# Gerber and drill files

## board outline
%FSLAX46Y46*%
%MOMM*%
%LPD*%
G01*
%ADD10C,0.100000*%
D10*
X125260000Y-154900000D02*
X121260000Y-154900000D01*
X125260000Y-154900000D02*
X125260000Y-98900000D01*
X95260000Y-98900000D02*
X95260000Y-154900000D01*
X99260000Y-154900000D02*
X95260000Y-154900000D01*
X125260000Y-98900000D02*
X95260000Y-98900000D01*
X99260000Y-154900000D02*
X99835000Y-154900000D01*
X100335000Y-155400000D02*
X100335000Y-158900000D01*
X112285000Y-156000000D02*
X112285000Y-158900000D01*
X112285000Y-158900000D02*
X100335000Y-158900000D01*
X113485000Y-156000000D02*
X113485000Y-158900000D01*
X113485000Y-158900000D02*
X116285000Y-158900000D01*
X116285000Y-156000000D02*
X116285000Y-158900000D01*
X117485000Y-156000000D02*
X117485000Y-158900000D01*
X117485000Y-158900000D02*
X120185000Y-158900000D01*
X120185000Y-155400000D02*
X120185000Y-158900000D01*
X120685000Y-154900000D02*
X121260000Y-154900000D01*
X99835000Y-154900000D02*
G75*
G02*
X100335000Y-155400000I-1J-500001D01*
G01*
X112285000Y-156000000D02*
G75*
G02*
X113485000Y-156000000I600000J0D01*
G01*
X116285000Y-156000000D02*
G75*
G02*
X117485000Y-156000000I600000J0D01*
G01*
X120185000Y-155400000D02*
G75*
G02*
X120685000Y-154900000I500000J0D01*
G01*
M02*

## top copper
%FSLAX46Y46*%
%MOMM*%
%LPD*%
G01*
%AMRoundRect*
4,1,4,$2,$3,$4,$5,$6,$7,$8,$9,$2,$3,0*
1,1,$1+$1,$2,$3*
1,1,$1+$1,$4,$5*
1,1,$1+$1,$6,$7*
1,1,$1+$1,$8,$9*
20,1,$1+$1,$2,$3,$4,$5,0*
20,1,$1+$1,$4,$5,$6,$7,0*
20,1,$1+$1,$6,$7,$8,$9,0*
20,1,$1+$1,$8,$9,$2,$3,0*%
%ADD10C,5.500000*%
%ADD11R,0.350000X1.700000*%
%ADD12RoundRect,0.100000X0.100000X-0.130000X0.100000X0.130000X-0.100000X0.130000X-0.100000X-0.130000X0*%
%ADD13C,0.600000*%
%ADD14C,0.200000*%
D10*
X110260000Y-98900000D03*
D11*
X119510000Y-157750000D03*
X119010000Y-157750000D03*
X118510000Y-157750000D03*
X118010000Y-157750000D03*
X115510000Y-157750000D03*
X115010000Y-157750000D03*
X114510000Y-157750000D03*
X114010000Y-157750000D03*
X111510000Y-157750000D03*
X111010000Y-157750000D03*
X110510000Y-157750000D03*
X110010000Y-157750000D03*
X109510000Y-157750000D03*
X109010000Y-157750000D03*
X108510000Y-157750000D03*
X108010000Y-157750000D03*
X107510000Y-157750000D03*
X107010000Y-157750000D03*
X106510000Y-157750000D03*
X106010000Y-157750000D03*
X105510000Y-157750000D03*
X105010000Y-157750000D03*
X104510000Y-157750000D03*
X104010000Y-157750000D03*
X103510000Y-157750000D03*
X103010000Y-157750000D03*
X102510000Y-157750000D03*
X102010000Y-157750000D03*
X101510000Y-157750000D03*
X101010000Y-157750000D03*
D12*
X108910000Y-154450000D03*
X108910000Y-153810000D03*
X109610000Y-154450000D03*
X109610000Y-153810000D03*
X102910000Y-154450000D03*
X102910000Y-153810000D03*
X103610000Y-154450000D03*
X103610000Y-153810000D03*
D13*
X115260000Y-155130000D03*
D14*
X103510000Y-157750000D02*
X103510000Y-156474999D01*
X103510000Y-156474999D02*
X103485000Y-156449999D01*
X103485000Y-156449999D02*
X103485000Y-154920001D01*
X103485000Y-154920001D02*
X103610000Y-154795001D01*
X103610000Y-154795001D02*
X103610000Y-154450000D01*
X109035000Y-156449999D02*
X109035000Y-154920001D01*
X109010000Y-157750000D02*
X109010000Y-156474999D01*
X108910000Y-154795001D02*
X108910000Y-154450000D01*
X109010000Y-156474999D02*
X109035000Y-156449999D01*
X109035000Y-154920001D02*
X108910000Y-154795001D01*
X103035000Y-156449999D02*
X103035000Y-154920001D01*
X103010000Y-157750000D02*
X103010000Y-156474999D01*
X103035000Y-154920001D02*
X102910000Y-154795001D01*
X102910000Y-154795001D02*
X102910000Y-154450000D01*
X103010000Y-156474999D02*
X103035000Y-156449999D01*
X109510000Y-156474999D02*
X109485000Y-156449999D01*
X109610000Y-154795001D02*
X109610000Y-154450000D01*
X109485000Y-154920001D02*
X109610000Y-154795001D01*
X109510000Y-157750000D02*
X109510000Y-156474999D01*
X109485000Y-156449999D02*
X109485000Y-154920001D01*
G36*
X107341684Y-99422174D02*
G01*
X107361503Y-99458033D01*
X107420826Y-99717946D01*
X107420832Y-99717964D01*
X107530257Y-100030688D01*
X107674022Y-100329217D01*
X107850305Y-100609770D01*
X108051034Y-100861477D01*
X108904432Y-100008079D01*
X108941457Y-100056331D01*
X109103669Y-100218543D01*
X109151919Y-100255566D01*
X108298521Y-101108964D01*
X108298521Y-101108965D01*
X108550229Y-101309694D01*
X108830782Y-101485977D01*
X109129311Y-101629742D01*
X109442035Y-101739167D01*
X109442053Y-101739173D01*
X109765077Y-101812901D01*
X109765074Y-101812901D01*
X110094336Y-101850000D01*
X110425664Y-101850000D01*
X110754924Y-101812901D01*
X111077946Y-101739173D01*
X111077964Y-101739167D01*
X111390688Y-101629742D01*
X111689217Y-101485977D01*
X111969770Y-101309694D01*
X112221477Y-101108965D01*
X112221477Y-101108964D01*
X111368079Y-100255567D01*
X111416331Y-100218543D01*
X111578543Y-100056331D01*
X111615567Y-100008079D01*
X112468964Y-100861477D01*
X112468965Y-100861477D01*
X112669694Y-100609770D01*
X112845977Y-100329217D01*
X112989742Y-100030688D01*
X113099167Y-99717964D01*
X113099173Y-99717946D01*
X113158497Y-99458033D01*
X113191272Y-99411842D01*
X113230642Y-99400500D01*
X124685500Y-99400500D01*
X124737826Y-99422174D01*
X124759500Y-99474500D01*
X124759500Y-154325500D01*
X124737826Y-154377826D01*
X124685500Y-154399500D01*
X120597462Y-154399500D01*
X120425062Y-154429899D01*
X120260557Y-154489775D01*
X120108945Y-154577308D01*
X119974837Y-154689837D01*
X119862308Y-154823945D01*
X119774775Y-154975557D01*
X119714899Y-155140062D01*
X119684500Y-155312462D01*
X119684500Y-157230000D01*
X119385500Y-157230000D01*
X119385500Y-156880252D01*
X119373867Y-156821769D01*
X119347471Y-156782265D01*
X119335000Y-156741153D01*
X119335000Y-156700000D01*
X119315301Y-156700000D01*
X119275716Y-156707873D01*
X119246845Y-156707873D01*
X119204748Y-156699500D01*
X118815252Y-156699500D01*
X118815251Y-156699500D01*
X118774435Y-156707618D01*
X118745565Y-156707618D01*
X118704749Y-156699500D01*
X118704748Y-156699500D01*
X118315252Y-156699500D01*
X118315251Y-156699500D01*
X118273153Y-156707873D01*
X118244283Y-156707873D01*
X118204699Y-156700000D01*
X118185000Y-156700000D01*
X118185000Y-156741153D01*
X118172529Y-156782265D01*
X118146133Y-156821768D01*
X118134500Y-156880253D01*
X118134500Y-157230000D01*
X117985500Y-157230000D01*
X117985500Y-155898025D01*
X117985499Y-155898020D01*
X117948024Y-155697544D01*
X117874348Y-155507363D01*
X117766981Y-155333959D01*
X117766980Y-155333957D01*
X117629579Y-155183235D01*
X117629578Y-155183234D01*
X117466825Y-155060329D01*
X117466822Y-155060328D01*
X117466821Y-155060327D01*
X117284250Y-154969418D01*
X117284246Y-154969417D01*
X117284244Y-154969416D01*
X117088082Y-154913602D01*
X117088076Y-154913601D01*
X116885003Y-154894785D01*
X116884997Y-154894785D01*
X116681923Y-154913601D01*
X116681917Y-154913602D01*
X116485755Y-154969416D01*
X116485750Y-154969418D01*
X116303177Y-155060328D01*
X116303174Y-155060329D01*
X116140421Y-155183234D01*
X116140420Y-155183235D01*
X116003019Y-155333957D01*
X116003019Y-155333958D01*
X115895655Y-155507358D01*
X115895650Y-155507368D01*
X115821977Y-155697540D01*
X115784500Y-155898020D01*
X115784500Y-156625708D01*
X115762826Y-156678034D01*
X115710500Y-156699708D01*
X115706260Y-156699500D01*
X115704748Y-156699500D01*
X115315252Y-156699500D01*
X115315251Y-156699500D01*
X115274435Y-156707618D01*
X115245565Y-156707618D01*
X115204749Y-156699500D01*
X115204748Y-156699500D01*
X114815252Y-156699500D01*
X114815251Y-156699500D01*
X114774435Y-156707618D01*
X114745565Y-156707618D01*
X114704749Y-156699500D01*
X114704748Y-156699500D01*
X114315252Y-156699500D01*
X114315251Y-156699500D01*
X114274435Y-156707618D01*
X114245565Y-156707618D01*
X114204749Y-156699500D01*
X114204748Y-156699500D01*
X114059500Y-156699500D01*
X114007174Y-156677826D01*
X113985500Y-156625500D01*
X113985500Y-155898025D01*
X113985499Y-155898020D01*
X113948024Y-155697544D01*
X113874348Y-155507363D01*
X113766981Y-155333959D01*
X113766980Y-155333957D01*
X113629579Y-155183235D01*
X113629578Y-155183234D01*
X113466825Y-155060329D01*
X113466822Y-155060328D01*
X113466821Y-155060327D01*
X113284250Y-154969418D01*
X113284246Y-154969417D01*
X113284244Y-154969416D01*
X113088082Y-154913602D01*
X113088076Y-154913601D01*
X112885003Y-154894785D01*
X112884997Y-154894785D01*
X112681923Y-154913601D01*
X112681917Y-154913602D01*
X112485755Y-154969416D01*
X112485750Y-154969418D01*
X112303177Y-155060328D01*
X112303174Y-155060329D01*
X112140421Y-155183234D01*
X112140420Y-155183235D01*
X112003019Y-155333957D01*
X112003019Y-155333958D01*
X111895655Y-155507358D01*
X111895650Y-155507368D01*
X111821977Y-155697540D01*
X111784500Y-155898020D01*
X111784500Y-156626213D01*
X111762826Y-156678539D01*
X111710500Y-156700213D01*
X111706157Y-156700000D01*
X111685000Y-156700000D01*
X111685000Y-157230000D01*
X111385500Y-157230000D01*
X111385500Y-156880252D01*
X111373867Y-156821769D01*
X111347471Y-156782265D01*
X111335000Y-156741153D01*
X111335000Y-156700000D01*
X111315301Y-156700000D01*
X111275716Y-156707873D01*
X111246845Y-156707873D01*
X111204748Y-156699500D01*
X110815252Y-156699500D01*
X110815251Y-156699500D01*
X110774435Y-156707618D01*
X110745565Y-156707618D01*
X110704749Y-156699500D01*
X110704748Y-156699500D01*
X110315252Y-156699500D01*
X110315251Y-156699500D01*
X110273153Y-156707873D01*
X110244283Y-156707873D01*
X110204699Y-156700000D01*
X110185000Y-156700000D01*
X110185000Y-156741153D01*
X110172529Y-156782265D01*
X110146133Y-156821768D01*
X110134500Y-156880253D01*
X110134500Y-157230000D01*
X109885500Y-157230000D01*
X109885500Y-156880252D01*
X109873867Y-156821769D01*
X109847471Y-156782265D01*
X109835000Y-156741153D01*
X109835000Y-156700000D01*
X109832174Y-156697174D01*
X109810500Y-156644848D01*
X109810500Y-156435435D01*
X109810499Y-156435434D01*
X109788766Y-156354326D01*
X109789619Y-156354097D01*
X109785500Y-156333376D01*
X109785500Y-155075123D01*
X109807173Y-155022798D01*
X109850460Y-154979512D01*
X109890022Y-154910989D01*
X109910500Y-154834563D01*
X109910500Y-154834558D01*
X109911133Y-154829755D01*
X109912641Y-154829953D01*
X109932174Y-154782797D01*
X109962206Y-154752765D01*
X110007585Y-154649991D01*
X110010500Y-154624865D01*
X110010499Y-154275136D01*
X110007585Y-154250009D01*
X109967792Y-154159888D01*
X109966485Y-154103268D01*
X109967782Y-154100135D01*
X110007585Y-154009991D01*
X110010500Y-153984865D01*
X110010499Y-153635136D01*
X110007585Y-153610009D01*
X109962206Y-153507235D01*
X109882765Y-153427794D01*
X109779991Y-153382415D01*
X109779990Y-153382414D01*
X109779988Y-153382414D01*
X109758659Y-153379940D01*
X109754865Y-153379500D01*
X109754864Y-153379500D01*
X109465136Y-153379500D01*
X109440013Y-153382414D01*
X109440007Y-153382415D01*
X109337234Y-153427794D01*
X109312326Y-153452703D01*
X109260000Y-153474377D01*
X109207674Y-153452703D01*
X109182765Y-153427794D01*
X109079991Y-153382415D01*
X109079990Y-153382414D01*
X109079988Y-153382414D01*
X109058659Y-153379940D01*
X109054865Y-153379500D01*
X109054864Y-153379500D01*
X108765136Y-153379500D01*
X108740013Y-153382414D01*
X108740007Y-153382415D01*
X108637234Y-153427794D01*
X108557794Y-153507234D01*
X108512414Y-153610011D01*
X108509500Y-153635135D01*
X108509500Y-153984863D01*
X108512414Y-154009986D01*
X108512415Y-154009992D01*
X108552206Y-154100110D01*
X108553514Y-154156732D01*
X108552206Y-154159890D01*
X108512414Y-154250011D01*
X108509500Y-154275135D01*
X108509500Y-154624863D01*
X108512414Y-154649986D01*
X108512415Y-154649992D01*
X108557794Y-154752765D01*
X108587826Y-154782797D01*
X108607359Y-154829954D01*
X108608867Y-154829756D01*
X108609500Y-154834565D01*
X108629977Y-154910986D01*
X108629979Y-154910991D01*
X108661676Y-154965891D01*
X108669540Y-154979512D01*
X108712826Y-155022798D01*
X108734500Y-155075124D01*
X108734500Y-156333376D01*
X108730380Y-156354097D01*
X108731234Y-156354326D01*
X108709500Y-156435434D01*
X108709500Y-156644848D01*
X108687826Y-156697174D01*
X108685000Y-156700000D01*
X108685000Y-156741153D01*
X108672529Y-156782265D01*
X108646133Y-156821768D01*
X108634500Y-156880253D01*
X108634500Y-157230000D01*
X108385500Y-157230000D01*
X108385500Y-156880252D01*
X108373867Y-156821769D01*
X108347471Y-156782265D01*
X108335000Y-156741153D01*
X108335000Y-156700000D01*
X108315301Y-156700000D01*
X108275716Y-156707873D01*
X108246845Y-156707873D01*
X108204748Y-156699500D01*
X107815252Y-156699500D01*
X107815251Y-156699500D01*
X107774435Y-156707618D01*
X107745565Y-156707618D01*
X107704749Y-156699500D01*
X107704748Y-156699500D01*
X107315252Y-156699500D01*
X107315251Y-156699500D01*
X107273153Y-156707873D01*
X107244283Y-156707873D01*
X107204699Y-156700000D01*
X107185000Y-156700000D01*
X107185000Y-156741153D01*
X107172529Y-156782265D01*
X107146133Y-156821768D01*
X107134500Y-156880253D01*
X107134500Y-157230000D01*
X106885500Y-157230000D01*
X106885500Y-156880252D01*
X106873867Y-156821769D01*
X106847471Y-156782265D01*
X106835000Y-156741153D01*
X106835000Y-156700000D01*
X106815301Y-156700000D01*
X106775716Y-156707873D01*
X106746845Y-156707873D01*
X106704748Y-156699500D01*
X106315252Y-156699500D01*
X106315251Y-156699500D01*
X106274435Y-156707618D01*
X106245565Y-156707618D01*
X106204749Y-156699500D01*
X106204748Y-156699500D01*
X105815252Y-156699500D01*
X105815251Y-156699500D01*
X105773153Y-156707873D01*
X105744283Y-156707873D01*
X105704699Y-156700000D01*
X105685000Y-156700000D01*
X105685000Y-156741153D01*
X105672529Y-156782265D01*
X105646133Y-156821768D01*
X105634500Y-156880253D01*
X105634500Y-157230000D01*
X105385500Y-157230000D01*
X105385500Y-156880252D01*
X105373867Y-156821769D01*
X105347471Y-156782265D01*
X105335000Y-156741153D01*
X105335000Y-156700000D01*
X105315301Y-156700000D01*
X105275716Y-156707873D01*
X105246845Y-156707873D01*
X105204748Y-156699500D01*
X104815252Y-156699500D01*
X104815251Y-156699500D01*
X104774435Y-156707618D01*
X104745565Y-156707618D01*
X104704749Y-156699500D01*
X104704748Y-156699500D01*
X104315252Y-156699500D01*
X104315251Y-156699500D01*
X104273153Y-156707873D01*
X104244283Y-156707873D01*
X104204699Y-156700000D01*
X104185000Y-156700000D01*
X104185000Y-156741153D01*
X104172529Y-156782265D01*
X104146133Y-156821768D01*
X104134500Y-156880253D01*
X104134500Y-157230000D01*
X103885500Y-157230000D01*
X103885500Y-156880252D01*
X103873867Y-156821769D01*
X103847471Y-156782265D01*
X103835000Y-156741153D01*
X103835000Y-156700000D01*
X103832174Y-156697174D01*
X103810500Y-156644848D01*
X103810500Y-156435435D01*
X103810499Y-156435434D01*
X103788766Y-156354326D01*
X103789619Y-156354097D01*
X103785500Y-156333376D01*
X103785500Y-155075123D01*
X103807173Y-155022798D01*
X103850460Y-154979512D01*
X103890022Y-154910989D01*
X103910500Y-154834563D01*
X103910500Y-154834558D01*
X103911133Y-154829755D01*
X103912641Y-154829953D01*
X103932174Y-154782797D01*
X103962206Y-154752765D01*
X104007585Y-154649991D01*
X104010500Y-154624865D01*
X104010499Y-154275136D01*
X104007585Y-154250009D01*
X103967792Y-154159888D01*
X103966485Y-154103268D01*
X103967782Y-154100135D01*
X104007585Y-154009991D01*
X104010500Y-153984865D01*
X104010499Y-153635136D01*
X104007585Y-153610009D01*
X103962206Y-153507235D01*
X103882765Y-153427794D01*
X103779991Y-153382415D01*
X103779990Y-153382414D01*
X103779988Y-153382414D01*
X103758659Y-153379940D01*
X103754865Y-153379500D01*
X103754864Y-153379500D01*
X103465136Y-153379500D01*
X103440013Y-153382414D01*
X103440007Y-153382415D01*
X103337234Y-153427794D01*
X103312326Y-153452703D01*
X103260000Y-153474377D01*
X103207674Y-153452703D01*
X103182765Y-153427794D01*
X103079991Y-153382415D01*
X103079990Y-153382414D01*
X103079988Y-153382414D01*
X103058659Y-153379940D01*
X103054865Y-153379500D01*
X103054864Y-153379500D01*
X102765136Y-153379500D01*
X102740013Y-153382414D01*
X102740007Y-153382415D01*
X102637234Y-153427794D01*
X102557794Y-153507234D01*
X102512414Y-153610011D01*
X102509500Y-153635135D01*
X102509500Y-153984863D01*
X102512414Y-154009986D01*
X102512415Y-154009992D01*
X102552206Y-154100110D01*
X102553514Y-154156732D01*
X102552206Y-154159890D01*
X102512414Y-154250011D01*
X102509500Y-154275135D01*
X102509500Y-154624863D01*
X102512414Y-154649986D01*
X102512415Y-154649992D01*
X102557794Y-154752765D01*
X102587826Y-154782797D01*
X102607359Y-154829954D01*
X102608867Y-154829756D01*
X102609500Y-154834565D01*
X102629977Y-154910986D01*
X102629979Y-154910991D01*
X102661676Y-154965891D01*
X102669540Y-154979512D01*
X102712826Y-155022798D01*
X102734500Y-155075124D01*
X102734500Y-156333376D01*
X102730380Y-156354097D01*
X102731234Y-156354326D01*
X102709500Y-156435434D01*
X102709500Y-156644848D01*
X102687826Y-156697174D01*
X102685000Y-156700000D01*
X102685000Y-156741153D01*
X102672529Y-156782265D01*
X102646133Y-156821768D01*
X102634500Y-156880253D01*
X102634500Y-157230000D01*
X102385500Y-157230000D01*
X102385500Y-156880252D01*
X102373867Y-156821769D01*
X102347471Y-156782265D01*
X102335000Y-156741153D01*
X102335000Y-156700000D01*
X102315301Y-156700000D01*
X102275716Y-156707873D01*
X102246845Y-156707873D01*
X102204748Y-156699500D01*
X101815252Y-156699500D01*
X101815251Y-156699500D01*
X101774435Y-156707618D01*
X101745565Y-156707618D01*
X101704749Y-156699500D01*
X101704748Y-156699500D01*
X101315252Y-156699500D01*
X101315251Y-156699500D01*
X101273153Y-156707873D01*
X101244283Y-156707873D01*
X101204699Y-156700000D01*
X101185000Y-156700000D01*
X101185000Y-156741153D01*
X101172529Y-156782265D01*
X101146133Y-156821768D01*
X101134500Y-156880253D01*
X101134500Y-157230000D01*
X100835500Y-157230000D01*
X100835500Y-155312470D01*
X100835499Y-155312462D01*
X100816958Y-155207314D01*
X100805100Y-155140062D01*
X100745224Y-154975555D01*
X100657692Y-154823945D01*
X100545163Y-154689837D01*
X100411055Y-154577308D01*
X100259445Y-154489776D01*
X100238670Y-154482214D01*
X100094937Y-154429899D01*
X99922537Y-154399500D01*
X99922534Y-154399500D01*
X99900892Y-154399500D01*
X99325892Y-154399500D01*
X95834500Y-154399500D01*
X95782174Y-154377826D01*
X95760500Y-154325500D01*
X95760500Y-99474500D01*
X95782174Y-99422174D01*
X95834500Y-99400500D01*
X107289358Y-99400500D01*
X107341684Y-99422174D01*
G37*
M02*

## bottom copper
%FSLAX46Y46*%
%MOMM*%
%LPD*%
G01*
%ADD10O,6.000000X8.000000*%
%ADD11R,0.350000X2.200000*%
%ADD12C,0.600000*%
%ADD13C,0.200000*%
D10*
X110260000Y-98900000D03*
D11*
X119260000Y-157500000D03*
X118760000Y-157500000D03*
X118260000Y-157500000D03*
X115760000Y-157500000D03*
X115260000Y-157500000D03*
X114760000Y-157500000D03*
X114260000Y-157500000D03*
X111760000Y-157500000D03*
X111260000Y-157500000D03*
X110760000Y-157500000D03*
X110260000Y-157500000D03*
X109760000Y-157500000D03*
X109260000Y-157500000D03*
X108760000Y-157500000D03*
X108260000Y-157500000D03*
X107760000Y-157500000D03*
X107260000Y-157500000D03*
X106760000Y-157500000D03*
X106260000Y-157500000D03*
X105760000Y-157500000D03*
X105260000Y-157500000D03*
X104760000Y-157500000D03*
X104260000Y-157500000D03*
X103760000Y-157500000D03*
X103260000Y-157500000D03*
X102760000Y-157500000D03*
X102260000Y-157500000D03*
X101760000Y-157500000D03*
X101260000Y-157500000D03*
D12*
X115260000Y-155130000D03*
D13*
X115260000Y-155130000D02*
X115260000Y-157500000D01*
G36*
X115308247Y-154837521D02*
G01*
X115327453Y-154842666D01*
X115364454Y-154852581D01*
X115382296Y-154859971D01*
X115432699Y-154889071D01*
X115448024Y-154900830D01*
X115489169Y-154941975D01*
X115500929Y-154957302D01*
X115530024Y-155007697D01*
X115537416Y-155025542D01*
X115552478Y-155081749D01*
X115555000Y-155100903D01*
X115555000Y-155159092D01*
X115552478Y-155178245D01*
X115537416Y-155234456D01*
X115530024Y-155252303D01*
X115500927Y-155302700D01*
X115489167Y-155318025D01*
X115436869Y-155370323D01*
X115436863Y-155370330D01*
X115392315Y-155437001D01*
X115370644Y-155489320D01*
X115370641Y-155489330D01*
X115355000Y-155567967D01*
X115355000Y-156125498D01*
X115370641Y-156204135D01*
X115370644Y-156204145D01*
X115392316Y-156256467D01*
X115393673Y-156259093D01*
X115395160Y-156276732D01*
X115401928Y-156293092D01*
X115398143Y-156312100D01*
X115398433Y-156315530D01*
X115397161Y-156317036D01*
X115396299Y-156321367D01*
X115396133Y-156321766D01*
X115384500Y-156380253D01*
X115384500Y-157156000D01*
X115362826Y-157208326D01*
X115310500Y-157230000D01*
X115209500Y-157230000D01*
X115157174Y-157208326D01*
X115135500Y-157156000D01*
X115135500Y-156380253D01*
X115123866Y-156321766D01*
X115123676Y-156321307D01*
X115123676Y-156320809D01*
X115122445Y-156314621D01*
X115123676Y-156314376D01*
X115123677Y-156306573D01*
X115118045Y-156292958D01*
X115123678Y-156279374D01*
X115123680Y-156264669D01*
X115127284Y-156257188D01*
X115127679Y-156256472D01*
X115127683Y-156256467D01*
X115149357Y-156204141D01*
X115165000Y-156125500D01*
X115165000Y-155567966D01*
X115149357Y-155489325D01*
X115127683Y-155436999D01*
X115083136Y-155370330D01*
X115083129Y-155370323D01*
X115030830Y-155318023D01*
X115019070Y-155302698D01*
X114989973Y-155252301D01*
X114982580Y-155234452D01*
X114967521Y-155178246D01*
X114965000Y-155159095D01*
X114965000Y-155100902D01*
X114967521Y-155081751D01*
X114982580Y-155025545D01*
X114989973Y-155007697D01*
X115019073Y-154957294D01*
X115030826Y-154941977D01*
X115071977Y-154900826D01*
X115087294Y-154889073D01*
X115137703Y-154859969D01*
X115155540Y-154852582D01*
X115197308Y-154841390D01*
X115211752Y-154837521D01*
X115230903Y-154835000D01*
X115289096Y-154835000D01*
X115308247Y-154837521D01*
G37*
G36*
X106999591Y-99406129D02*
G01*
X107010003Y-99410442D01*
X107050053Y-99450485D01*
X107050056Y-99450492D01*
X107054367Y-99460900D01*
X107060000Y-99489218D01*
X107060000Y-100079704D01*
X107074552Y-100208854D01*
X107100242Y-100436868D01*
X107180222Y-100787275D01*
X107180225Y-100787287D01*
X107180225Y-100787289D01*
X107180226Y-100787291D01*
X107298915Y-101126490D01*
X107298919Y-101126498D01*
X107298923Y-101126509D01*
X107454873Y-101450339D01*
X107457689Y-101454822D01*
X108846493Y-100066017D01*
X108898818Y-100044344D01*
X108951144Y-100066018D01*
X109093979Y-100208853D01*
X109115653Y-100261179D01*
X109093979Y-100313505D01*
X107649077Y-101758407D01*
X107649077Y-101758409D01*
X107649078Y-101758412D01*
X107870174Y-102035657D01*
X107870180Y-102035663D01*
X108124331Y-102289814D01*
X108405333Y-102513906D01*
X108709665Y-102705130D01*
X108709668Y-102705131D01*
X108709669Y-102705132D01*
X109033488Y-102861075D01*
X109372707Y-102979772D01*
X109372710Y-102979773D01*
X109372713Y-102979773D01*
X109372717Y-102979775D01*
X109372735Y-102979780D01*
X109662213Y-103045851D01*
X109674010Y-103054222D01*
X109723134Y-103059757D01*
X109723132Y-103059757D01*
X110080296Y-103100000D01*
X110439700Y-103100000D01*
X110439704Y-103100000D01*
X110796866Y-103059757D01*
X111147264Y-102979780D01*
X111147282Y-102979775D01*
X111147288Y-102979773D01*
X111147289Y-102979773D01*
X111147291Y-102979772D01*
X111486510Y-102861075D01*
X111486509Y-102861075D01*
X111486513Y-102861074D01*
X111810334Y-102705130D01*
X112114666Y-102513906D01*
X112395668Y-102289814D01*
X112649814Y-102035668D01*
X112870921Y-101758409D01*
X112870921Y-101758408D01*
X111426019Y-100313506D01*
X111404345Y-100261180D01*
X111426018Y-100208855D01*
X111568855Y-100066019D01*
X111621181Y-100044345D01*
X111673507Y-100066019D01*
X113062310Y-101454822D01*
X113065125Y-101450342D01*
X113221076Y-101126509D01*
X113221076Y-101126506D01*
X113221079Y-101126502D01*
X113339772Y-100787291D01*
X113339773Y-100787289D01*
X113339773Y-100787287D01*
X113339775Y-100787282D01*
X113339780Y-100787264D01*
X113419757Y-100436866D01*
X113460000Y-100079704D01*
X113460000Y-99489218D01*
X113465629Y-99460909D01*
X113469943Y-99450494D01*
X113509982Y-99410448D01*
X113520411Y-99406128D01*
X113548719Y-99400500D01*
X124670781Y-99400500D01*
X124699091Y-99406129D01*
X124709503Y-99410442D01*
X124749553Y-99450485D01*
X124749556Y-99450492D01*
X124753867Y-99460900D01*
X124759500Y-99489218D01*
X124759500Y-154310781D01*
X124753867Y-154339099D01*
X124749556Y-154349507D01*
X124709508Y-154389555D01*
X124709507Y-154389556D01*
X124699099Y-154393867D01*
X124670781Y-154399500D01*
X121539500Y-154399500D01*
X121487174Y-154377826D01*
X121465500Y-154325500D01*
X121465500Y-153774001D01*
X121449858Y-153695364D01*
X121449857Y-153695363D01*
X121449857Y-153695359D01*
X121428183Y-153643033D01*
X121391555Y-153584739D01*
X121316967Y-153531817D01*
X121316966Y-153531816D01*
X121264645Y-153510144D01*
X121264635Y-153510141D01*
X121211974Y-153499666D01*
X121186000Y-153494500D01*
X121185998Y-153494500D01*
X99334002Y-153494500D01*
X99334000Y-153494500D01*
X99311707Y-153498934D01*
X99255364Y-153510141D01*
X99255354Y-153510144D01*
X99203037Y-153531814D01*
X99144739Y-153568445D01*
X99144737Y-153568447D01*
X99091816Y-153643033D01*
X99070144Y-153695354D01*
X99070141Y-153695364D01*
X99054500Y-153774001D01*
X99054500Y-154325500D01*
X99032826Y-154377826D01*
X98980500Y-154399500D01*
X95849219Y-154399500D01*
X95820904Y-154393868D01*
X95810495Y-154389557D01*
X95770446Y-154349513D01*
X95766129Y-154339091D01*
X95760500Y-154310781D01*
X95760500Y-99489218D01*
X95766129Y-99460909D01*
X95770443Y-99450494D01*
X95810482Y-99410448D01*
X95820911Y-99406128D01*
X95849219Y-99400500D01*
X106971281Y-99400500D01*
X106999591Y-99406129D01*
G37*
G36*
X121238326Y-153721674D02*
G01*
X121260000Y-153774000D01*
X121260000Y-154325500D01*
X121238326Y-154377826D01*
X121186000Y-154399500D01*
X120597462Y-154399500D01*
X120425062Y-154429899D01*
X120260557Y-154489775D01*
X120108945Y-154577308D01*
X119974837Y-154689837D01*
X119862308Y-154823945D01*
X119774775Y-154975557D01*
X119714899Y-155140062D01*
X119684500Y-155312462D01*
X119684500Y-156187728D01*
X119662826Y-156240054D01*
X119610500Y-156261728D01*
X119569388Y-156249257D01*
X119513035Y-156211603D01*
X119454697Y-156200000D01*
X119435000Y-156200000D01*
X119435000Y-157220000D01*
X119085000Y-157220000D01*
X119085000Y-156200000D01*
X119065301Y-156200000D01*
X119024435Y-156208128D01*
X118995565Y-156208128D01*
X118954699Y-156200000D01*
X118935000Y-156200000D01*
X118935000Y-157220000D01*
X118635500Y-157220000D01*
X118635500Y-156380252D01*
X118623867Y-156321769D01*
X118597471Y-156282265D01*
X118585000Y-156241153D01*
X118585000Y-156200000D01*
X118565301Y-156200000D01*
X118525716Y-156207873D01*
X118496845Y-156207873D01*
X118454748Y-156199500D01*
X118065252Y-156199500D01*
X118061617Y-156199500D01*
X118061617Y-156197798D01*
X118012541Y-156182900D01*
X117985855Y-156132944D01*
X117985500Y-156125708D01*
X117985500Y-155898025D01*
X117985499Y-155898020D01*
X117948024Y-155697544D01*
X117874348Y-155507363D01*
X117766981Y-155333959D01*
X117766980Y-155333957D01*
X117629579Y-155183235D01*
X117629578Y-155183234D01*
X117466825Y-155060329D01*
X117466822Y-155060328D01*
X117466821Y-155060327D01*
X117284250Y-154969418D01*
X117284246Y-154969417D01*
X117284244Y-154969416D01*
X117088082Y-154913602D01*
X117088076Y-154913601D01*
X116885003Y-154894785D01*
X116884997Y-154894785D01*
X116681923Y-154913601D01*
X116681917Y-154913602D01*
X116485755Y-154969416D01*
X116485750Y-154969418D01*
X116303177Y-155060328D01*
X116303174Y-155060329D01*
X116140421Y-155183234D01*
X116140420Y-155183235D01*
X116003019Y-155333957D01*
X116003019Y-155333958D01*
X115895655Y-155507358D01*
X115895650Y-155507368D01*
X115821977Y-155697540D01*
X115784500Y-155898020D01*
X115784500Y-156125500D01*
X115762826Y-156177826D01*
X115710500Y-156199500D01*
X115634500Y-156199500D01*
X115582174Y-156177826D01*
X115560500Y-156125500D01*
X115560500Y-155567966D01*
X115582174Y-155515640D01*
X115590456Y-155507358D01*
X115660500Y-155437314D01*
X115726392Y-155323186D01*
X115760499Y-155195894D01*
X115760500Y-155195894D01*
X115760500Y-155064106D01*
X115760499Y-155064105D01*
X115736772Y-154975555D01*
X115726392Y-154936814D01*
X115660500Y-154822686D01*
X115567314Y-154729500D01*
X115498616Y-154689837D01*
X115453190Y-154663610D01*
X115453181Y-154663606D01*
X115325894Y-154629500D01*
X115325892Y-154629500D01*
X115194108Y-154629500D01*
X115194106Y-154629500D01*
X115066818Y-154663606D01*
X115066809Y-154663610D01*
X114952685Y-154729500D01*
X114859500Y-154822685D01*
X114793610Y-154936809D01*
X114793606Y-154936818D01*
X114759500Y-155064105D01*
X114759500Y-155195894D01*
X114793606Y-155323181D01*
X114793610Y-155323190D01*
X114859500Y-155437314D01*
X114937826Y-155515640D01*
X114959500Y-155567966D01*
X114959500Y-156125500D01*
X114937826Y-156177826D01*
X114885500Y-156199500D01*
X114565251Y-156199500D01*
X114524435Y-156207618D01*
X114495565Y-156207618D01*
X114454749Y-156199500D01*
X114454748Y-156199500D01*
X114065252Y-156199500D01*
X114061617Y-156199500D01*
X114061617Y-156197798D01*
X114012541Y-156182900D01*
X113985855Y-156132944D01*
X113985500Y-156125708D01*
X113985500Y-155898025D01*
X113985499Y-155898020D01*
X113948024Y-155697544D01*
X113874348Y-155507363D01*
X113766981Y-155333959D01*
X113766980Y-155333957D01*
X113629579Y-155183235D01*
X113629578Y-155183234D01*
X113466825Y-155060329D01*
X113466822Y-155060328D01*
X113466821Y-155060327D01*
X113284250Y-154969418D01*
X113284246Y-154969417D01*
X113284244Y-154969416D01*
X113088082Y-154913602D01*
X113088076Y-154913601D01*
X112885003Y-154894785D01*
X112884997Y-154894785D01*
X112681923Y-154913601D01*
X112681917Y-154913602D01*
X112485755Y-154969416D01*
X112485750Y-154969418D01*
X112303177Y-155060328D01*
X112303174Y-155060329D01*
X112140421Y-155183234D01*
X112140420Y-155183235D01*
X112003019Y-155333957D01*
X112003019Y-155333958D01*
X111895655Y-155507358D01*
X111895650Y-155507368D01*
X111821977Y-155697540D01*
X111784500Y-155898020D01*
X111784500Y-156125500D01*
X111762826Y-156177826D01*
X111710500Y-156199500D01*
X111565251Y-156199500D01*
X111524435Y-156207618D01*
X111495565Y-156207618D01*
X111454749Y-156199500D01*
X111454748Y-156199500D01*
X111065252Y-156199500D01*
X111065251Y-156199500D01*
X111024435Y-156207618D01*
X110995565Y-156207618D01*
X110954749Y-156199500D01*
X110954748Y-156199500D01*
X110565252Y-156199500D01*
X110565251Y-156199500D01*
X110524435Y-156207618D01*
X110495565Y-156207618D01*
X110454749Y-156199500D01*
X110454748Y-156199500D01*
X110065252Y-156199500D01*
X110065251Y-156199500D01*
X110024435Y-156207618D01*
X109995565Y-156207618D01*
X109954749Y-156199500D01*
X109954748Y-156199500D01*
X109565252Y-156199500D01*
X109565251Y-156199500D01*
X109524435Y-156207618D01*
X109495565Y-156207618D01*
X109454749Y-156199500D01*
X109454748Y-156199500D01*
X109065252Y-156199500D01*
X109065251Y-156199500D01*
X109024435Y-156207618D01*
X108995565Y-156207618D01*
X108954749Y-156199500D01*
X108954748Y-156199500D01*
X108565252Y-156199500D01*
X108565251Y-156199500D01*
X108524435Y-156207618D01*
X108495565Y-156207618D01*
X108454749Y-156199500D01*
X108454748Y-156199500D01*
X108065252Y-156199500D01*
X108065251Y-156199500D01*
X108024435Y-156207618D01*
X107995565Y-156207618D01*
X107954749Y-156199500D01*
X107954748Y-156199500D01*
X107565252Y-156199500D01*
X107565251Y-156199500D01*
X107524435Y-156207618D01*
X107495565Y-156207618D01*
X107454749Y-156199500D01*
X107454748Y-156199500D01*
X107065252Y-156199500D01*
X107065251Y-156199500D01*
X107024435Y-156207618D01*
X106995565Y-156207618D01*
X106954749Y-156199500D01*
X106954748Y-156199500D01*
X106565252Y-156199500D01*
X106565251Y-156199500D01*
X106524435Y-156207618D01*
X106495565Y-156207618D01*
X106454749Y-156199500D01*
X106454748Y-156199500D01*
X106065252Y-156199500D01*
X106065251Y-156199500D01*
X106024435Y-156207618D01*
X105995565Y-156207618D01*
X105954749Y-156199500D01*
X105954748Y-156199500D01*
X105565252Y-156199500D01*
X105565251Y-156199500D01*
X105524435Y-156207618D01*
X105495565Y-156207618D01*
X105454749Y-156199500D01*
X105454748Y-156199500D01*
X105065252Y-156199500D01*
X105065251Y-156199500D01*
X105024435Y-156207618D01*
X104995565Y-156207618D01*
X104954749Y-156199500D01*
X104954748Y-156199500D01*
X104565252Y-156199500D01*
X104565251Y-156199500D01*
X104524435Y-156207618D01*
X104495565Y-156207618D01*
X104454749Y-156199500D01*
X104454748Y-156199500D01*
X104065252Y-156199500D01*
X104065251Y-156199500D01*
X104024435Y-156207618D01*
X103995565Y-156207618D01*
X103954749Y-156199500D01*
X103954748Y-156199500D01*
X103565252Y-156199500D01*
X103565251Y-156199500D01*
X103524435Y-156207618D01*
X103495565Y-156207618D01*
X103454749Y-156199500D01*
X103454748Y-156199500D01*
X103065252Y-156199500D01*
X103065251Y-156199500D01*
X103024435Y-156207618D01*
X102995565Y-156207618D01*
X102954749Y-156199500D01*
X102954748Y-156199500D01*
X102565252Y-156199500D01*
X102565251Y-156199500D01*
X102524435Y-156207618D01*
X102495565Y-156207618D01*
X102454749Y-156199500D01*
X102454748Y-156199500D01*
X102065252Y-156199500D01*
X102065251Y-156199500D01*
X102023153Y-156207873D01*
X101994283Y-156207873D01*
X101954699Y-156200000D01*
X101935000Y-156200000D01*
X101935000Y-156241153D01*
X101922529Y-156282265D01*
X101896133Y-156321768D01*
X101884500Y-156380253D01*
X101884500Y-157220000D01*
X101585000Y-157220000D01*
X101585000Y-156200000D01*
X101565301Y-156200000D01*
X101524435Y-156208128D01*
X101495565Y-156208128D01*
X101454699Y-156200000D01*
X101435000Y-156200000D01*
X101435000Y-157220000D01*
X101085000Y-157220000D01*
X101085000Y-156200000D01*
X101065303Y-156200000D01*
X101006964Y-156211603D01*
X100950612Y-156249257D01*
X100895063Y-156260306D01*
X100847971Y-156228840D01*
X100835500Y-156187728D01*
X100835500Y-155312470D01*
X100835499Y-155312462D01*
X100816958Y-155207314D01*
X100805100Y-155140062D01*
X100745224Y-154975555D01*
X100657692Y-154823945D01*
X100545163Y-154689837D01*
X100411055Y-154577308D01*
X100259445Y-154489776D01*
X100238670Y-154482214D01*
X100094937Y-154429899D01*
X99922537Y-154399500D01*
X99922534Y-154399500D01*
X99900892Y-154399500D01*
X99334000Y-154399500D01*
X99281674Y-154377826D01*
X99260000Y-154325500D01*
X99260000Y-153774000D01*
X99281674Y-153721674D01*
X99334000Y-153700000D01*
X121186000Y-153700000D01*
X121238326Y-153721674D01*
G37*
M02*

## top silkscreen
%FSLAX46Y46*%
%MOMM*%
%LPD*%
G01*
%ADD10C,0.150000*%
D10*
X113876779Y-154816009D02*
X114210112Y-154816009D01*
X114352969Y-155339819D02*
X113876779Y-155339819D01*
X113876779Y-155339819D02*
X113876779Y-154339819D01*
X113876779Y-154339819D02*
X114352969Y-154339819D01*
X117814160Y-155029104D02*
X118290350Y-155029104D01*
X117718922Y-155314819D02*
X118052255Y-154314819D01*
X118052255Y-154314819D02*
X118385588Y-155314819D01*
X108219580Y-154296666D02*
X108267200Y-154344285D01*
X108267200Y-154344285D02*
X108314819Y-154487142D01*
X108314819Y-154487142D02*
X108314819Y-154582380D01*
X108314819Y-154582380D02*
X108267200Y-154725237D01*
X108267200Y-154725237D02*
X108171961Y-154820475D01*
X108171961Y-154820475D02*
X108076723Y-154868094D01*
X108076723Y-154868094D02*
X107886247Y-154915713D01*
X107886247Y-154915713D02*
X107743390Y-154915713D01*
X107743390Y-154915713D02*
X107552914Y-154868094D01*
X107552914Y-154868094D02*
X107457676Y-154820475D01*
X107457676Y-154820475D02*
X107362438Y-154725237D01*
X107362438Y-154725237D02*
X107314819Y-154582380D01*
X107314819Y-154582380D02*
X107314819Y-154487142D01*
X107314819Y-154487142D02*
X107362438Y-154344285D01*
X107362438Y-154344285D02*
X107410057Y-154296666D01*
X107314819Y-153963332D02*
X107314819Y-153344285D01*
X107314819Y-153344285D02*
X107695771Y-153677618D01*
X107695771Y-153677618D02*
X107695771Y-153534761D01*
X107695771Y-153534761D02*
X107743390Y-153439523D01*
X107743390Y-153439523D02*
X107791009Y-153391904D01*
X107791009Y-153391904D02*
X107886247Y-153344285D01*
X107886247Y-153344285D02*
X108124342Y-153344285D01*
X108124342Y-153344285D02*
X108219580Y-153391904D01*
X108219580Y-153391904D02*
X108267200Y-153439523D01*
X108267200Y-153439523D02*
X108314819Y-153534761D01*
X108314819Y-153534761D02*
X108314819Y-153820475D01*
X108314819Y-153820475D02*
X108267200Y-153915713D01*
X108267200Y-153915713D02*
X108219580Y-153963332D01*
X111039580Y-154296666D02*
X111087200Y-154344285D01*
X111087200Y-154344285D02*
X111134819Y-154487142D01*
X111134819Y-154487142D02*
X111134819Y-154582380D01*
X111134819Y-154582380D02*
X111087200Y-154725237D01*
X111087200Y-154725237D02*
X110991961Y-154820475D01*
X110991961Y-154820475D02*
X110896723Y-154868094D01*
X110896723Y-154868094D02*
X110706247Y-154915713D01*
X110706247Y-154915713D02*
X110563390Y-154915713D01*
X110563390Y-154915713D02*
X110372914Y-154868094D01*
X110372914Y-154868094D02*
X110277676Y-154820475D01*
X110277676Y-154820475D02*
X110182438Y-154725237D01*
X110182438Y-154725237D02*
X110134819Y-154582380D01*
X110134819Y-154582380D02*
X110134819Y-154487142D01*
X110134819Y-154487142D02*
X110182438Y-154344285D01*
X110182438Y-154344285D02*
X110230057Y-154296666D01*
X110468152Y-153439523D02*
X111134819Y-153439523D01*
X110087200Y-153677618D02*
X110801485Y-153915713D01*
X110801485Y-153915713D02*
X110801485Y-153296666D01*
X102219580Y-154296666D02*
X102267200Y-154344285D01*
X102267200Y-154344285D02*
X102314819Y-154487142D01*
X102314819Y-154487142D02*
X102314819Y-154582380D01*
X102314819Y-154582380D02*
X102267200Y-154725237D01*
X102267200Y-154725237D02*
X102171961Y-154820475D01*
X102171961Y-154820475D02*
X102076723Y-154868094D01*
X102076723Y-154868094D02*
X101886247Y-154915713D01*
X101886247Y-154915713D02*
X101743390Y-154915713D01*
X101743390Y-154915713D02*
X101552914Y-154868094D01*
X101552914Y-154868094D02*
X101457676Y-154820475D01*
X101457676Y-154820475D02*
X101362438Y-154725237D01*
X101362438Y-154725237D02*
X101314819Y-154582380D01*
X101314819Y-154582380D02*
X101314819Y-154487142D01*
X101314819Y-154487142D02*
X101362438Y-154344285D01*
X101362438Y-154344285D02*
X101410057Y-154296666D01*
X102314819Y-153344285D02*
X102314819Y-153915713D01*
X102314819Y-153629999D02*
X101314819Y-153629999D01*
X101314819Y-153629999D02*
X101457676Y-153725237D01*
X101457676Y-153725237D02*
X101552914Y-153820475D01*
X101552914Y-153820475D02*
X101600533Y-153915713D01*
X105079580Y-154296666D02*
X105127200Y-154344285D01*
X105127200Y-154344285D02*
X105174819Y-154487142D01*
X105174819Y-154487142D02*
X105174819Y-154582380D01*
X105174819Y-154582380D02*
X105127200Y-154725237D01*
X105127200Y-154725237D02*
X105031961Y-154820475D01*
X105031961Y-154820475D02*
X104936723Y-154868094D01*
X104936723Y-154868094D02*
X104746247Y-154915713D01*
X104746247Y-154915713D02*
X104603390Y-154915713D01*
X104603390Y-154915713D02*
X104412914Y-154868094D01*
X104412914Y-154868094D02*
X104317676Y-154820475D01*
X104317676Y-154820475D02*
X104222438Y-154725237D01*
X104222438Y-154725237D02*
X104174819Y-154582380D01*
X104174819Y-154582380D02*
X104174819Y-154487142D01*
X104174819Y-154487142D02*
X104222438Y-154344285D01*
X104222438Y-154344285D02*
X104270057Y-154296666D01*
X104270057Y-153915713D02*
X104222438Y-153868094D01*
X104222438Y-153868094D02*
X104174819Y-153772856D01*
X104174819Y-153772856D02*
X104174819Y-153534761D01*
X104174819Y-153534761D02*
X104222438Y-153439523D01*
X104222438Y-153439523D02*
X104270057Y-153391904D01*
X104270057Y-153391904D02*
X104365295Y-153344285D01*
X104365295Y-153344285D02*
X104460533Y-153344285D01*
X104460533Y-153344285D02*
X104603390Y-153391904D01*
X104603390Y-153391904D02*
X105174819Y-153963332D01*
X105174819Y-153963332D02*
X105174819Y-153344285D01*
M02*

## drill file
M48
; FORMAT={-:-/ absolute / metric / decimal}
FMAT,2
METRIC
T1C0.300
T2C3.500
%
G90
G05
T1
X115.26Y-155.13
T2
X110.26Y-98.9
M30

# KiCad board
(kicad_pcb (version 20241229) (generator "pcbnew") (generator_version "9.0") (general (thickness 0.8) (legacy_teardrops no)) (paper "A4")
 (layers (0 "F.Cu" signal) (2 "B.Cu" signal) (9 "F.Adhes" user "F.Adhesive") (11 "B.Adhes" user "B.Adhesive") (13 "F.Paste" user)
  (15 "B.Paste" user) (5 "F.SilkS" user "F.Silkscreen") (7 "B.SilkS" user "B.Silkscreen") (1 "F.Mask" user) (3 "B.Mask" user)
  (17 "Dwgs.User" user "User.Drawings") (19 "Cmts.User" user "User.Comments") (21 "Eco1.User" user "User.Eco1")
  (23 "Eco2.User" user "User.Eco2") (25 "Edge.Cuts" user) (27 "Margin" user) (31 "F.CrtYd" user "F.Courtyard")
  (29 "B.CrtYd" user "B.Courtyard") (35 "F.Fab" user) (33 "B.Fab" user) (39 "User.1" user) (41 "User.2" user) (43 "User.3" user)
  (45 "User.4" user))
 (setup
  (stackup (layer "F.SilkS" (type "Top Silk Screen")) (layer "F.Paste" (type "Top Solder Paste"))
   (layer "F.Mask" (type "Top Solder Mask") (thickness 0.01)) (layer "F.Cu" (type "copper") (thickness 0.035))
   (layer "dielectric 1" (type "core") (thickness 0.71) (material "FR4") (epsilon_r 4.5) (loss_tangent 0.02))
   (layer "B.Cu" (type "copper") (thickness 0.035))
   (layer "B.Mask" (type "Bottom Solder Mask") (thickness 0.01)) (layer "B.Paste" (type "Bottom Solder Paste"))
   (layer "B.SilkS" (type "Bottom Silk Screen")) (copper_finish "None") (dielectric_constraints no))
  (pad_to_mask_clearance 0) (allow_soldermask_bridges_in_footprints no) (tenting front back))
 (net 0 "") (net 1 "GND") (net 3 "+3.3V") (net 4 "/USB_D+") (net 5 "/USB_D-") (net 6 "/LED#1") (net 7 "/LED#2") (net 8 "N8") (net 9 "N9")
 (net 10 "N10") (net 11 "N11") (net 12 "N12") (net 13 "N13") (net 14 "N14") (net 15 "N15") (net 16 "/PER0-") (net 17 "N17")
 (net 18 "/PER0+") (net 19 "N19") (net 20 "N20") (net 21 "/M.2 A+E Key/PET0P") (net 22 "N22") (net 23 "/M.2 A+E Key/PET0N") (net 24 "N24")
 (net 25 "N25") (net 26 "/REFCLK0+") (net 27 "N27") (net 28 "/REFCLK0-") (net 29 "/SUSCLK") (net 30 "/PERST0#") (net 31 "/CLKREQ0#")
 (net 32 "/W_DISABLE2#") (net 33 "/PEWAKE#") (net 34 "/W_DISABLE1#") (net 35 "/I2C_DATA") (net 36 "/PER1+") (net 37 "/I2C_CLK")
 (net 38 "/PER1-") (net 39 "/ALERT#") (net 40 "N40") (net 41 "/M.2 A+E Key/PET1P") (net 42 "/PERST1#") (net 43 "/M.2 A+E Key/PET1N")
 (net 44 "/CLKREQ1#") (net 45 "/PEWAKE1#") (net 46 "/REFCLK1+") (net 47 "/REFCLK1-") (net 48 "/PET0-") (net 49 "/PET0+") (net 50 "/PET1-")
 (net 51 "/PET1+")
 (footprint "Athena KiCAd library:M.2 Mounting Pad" (layer "F.Cu") (at 110.26 98.9)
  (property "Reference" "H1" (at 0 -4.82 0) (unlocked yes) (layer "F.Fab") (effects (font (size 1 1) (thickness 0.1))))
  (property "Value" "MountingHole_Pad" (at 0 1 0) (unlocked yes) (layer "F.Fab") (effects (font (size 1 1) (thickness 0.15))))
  (pad "1" thru_hole circle (at 0 0) (size 5.5 5.5) (drill 3.5) (layers "*.Cu" "*.Mask") (remove_unused_layers no) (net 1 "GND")
   (padstack (mode front_inner_back)
    (layer "Inner" (shape circle) (size 5.5 5.5) (zone_connect -1))
    (layer "B.Cu" (shape oval) (size 6 8) (thermal_bridge_angle 45) (zone_connect -1)))))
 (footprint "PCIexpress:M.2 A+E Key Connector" (layer "F.Cu") (at 110.26 157.79)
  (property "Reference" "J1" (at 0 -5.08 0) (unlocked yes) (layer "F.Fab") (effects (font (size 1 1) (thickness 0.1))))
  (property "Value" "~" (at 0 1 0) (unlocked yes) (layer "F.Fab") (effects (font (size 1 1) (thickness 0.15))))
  (fp_line (start -11 -2.89) (end -10.425 -2.89) (stroke (width 0.1) (type default)) (layer "Edge.Cuts") (net 2))
  (fp_line (start -9.925 -2.39) (end -9.925 1.11) (stroke (width 0.1) (type default)) (layer "Edge.Cuts") (net 2))
  (fp_line (start 2.025 -1.79) (end 2.025 1.11) (stroke (width 0.1) (type default)) (layer "Edge.Cuts") (net 2))
  (fp_line (start 2.025 1.11) (end -9.925 1.11) (stroke (width 0.1) (type default)) (layer "Edge.Cuts") (net 2))
  (fp_line (start 3.225 -1.79) (end 3.225 1.11) (stroke (width 0.1) (type default)) (layer "Edge.Cuts") (net 2))
  (fp_line (start 3.225 1.11) (end 6.025 1.11) (stroke (width 0.1) (type default)) (layer "Edge.Cuts") (net 2))
  (fp_line (start 6.025 -1.79) (end 6.025 1.11) (stroke (width 0.1) (type default)) (layer "Edge.Cuts") (net 2))
  (fp_line (start 7.225 -1.79) (end 7.225 1.11) (stroke (width 0.1) (type default)) (layer "Edge.Cuts") (net 2))
  (fp_line (start 7.225 1.11) (end 9.925 1.11) (stroke (width 0.1) (type default)) (layer "Edge.Cuts") (net 2))
  (fp_line (start 9.925 -2.39) (end 9.925 1.11) (stroke (width 0.1) (type default)) (layer "Edge.Cuts") (net 2))
  (fp_line (start 10.425 -2.89) (end 11 -2.89) (stroke (width 0.1) (type default)) (layer "Edge.Cuts") (net 2))
  (fp_arc (start -10.425 -2.89) (mid -10.071447 -2.743553) (end -9.925 -2.39) (stroke (width 0.1) (type default)) (layer "Edge.Cuts")
   (net 2))
  (fp_arc (start 2.025 -1.79) (mid 2.625 -2.39) (end 3.225 -1.79) (stroke (width 0.1) (type default)) (layer "Edge.Cuts") (net 2))
  (fp_arc (start 6.025 -1.79) (mid 6.625 -2.39) (end 7.225 -1.79) (stroke (width 0.1) (type default)) (layer "Edge.Cuts") (net 2))
  (fp_arc (start 9.925 -2.39) (mid 10.071447 -2.743553) (end 10.425 -2.89) (stroke (width 0.1) (type default)) (layer "Edge.Cuts") (net 2))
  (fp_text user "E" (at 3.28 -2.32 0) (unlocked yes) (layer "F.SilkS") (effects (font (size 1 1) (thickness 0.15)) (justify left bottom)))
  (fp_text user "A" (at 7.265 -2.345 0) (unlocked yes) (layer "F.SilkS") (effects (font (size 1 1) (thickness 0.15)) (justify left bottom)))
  (pad "1" smd rect (at 9.25 -0.04 180) (size 0.35 1.7) (layers "F.Cu") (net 1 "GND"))
  (pad "2" smd rect (at 9 -0.29 180) (size 0.35 2.2) (layers "B.Cu") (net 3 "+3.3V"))
  (pad "3" smd rect (at 8.75 -0.04 180) (size 0.35 1.7) (layers "F.Cu") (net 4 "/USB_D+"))
  (pad "4" smd rect (at 8.5 -0.29 180) (size 0.35 2.2) (layers "B.Cu") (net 3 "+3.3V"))
  (pad "5" smd rect (at 8.25 -0.04 180) (size 0.35 1.7) (layers "F.Cu") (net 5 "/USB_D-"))
  (pad "6" smd rect (at 8 -0.29 180) (size 0.35 2.2) (layers "B.Cu") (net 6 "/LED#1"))
  (pad "7" smd rect (at 7.75 -0.04 180) (size 0.35 1.7) (layers "F.Cu") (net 1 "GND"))
  (pad "16" smd rect (at 5.5 -0.29 180) (size 0.35 2.2) (layers "B.Cu") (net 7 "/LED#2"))
  (pad "17" smd rect (at 5.25 -0.04 180) (size 0.35 1.7) (layers "F.Cu") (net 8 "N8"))
  (pad "18" smd rect (at 5 -0.29 180) (size 0.35 2.2) (layers "B.Cu") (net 1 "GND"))
  (pad "19" smd rect (at 4.75 -0.04 180) (size 0.35 1.7) (layers "F.Cu") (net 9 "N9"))
  (pad "20" smd rect (at 4.5 -0.29 180) (size 0.35 2.2) (layers "B.Cu") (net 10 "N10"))
  (pad "21" smd rect (at 4.25 -0.04 180) (size 0.35 1.7) (layers "F.Cu") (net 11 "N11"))
  (pad "22" smd rect (at 4 -0.29 180) (size 0.35 2.2) (layers "B.Cu") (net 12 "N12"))
  (pad "23" smd rect (at 3.75 -0.04 180) (size 0.35 1.7) (layers "F.Cu") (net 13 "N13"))
  (pad "32" smd rect (at 1.5 -0.29 180) (size 0.35 2.2) (layers "B.Cu") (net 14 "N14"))
  (pad "33" smd rect (at 1.25 -0.04 180) (size 0.35 1.7) (layers "F.Cu") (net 1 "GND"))
  (pad "34" smd rect (at 1 -0.29 180) (size 0.35 2.2) (layers "B.Cu") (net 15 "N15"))
  (pad "35" smd rect (at 0.75 -0.04 180) (size 0.35 1.7) (layers "F.Cu") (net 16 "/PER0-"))
  (pad "36" smd rect (at 0.5 -0.29 180) (size 0.35 2.2) (layers "B.Cu") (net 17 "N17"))
  (pad "37" smd rect (at 0.25 -0.04 180) (size 0.35 1.7) (layers "F.Cu") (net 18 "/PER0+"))
  (pad "38" smd rect (at 0 -0.29 180) (size 0.35 2.2) (layers "B.Cu") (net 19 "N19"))
  (pad "39" smd rect (at -0.25 -0.04 180) (size 0.35 1.7) (layers "F.Cu") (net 1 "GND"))
  (pad "40" smd rect (at -0.5 -0.29 180) (size 0.35 2.2) (layers "B.Cu") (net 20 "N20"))
  (pad "41" smd rect (at -0.75 -0.04 180) (size 0.35 1.7) (layers "F.Cu") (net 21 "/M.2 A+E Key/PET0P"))
  (pad "42" smd rect (at -1 -0.29 180) (size 0.35 2.2) (layers "B.Cu") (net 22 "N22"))
  (pad "43" smd rect (at -1.25 -0.04 180) (size 0.35 1.7) (layers "F.Cu") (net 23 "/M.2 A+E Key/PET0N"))
  (pad "44" smd rect (at -1.5 -0.29 180) (size 0.35 2.2) (layers "B.Cu") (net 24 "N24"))
  (pad "45" smd rect (at -1.75 -0.04 180) (size 0.35 1.7) (layers "F.Cu") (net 1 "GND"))
  (pad "46" smd rect (at -2 -0.29 180) (size 0.35 2.2) (layers "B.Cu") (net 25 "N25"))
  (pad "47" smd rect (at -2.25 -0.04 180) (size 0.35 1.7) (layers "F.Cu") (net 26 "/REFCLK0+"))
  (pad "48" smd rect (at -2.5 -0.29 180) (size 0.35 2.2) (layers "B.Cu") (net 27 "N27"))
  (pad "49" smd rect (at -2.75 -0.04 180) (size 0.35 1.7) (layers "F.Cu") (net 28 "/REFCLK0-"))
  (pad "50" smd rect (at -3 -0.29 180) (size 0.35 2.2) (layers "B.Cu") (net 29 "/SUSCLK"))
  (pad "51" smd rect (at -3.25 -0.04 180) (size 0.35 1.7) (layers "F.Cu") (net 1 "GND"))
  (pad "52" smd rect (at -3.5 -0.29 180) (size 0.35 2.2) (layers "B.Cu") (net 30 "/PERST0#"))
  (pad "53" smd rect (at -3.75 -0.04 180) (size 0.35 1.7) (layers "F.Cu") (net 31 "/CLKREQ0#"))
  (pad "54" smd rect (at -4 -0.29 180) (size 0.35 2.2) (layers "B.Cu") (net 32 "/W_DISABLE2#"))
  (pad "55" smd rect (at -4.25 -0.04 180) (size 0.35 1.7) (layers "F.Cu") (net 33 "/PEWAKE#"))
  (pad "56" smd rect (at -4.5 -0.29 180) (size 0.35 2.2) (layers "B.Cu") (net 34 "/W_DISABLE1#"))
  (pad "57" smd rect (at -4.75 -0.04 180) (size 0.35 1.7) (layers "F.Cu") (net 1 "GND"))
  (pad "58" smd rect (at -5 -0.29 180) (size 0.35 2.2) (layers "B.Cu") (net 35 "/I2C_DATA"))
  (pad "59" smd rect (at -5.25 -0.04 180) (size 0.35 1.7) (layers "F.Cu") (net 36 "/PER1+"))
  (pad "60" smd rect (at -5.5 -0.29 180) (size 0.35 2.2) (layers "B.Cu") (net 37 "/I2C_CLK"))
  (pad "61" smd rect (at -5.75 -0.04 180) (size 0.35 1.7) (layers "F.Cu") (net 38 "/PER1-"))
  (pad "62" smd rect (at -6 -0.29 180) (size 0.35 2.2) (layers "B.Cu") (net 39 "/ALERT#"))
  (pad "63" smd rect (at -6.25 -0.04 180) (size 0.35 1.7) (layers "F.Cu") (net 1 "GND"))
  (pad "64" smd rect (at -6.5 -0.29 180) (size 0.35 2.2) (layers "B.Cu") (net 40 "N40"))
  (pad "65" smd rect (at -6.75 -0.04 180) (size 0.35 1.7) (layers "F.Cu") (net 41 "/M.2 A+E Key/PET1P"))
  (pad "66" smd rect (at -7 -0.29 180) (size 0.35 2.2) (layers "B.Cu") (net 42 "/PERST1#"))
  (pad "67" smd rect (at -7.25 -0.04 180) (size 0.35 1.7) (layers "F.Cu") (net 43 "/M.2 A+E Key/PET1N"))
  (pad "68" smd rect (at -7.5 -0.29 180) (size 0.35 2.2) (layers "B.Cu") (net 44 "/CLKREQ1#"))
  (pad "69" smd rect (at -7.75 -0.04 180) (size 0.35 1.7) (layers "F.Cu") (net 1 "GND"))
  (pad "70" smd rect (at -8 -0.29 180) (size 0.35 2.2) (layers "B.Cu") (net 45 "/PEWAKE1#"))
  (pad "71" smd rect (at -8.25 -0.04 180) (size 0.35 1.7) (layers "F.Cu") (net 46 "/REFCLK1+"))
  (pad "72" smd rect (at -8.5 -0.29 180) (size 0.35 2.2) (layers "B.Cu") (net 3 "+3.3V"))
  (pad "73" smd rect (at -8.75 -0.04 180) (size 0.35 1.7) (layers "F.Cu") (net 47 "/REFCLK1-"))
  (pad "74" smd rect (at -9 -0.29 180) (size 0.35 2.2) (layers "B.Cu") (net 3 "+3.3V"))
  (pad "75" smd rect (at -9.25 -0.04 180) (size 0.35 1.7) (layers "F.Cu") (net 1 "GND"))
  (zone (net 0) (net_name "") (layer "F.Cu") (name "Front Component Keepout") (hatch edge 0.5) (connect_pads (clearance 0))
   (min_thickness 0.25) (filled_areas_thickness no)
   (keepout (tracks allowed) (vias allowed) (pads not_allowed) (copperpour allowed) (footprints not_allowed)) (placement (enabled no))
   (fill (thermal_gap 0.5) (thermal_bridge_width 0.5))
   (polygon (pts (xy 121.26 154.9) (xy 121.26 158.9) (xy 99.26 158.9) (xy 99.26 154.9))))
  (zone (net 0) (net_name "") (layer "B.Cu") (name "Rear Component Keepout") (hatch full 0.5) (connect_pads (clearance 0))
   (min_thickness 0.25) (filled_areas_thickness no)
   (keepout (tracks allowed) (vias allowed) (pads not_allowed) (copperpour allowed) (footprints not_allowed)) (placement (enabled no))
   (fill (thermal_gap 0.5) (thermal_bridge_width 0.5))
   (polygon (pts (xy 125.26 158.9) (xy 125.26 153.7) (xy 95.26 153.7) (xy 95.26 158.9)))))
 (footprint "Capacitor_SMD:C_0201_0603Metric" (layer "F.Cu") (at 108.91 154.13 90)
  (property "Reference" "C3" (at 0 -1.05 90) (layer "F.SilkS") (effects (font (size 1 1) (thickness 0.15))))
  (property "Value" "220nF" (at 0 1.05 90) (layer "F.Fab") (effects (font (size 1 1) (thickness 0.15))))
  (pad "" smd roundrect (at -0.345 0 90) (size 0.318 0.36) (layers "F.Paste") (roundrect_rratio 0.25))
  (pad "" smd roundrect (at 0.345 0 90) (size 0.318 0.36) (layers "F.Paste") (roundrect_rratio 0.25))
  (pad "1" smd roundrect (at -0.32 0 90) (size 0.46 0.4) (layers "F.Cu" "F.Mask") (roundrect_rratio 0.25) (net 23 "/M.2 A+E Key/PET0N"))
  (pad "2" smd roundrect (at 0.32 0 90) (size 0.46 0.4) (layers "F.Cu" "F.Mask") (roundrect_rratio 0.25) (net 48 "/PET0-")))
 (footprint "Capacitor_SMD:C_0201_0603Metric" (layer "F.Cu") (at 109.61 154.13 90)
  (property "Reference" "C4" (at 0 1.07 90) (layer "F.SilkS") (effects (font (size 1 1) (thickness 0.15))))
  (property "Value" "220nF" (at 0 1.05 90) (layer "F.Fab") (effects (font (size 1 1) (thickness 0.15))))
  (pad "" smd roundrect (at -0.345 0 90) (size 0.318 0.36) (layers "F.Paste") (roundrect_rratio 0.25))
  (pad "" smd roundrect (at 0.345 0 90) (size 0.318 0.36) (layers "F.Paste") (roundrect_rratio 0.25))
  (pad "1" smd roundrect (at -0.32 0 90) (size 0.46 0.4) (layers "F.Cu" "F.Mask") (roundrect_rratio 0.25) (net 21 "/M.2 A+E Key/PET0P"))
  (pad "2" smd roundrect (at 0.32 0 90) (size 0.46 0.4) (layers "F.Cu" "F.Mask") (roundrect_rratio 0.25) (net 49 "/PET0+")))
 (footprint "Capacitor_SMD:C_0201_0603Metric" (layer "F.Cu") (at 102.91 154.13 90)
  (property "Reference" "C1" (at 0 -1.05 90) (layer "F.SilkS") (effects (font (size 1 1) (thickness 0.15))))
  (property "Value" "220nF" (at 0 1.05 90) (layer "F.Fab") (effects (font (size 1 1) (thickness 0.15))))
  (pad "" smd roundrect (at -0.345 0 90) (size 0.318 0.36) (layers "F.Paste") (roundrect_rratio 0.25))
  (pad "" smd roundrect (at 0.345 0 90) (size 0.318 0.36) (layers "F.Paste") (roundrect_rratio 0.25))
  (pad "1" smd roundrect (at -0.32 0 90) (size 0.46 0.4) (layers "F.Cu" "F.Mask") (roundrect_rratio 0.25) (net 43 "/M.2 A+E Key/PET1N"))
  (pad "2" smd roundrect (at 0.32 0 90) (size 0.46 0.4) (layers "F.Cu" "F.Mask") (roundrect_rratio 0.25) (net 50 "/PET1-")))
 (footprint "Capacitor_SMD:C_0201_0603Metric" (layer "F.Cu") (at 103.61 154.13 90)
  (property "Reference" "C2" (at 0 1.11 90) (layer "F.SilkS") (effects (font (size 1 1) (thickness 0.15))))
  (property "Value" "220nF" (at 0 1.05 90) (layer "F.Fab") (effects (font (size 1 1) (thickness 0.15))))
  (pad "" smd roundrect (at -0.345 0 90) (size 0.318 0.36) (layers "F.Paste") (roundrect_rratio 0.25))
  (pad "" smd roundrect (at 0.345 0 90) (size 0.318 0.36) (layers "F.Paste") (roundrect_rratio 0.25))
  (pad "1" smd roundrect (at -0.32 0 90) (size 0.46 0.4) (layers "F.Cu" "F.Mask") (roundrect_rratio 0.25) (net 41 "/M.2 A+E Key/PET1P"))
  (pad "2" smd roundrect (at 0.32 0 90) (size 0.46 0.4) (layers "F.Cu" "F.Mask") (roundrect_rratio 0.25) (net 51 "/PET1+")))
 (gr_line (start 125.26 154.9) (end 121.26 154.9) (stroke (width 0.1) (type default)) (layer "Edge.Cuts"))
 (gr_line (start 125.26 154.9) (end 125.26 98.9) (stroke (width 0.1) (type default)) (layer "Edge.Cuts"))
 (gr_line (start 95.26 98.9) (end 95.26 154.9) (stroke (width 0.1) (type default)) (layer "Edge.Cuts"))
 (gr_line (start 99.26 154.9) (end 95.26 154.9) (stroke (width 0.1) (type default)) (layer "Edge.Cuts"))
 (gr_line (start 125.26 98.9) (end 95.26 98.9) (stroke (width 0.1) (type default)) (layer "Edge.Cuts"))
 (via (at 115.26 155.13) (size 0.6) (drill 0.3) (layers "F.Cu" "B.Cu") (free yes) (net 1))
 (segment (start 115.26 155.13) (end 115.26 157.5) (width 0.2) (layer "B.Cu") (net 1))
 (segment (start 103.51 157.75) (end 103.51 156.474999) (width 0.2) (layer "F.Cu") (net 41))
 (segment (start 103.51 156.474999) (end 103.485 156.449999) (width 0.2) (layer "F.Cu") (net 41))
 (segment (start 103.485 156.449999) (end 103.485 154.920001) (width 0.2) (layer "F.Cu") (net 41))
 (segment (start 103.485 154.920001) (end 103.61 154.795001) (width 0.2) (layer "F.Cu") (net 41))
 (segment (start 103.61 154.795001) (end 103.61 154.45) (width 0.2) (layer "F.Cu") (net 41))
 (segment (start 109.035 156.449999) (end 109.035 154.920001) (width 0.2) (layer "F.Cu") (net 23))
 (segment (start 109.01 157.75) (end 109.01 156.474999) (width 0.2) (layer "F.Cu") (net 23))
 (segment (start 108.91 154.795001) (end 108.91 154.45) (width 0.2) (layer "F.Cu") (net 23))
 (segment (start 109.01 156.474999) (end 109.035 156.449999) (width 0.2) (layer "F.Cu") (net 23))
 (segment (start 109.035 154.920001) (end 108.91 154.795001) (width 0.2) (layer "F.Cu") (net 23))
 (segment (start 103.035 156.449999) (end 103.035 154.920001) (width 0.2) (layer "F.Cu") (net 43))
 (segment (start 103.01 157.75) (end 103.01 156.474999) (width 0.2) (layer "F.Cu") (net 43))
 (segment (start 103.035 154.920001) (end 102.91 154.795001) (width 0.2) (layer "F.Cu") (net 43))
 (segment (start 102.91 154.795001) (end 102.91 154.45) (width 0.2) (layer "F.Cu") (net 43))
 (segment (start 103.01 156.474999) (end 103.035 156.449999) (width 0.2) (layer "F.Cu") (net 43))
 (segment (start 109.51 156.474999) (end 109.485 156.449999) (width 0.2) (layer "F.Cu") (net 21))
 (segment (start 109.61 154.795001) (end 109.61 154.45) (width 0.2) (layer "F.Cu") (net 21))
 (segment (start 109.485 154.920001) (end 109.61 154.795001) (width 0.2) (layer "F.Cu") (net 21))
 (segment (start 109.51 157.75) (end 109.51 156.474999) (width 0.2) (layer "F.Cu") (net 21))
 (segment (start 109.485 156.449999) (end 109.485 154.920001) (width 0.2) (layer "F.Cu") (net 21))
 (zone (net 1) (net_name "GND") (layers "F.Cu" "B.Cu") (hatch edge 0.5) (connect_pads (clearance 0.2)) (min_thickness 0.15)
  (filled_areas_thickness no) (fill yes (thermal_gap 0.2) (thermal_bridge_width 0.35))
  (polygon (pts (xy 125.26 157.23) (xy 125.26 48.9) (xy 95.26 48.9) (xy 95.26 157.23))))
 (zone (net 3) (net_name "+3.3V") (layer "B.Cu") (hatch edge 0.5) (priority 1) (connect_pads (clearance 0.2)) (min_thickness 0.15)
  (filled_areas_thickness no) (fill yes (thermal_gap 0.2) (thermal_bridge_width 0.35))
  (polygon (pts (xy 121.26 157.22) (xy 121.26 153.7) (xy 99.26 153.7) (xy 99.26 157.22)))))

